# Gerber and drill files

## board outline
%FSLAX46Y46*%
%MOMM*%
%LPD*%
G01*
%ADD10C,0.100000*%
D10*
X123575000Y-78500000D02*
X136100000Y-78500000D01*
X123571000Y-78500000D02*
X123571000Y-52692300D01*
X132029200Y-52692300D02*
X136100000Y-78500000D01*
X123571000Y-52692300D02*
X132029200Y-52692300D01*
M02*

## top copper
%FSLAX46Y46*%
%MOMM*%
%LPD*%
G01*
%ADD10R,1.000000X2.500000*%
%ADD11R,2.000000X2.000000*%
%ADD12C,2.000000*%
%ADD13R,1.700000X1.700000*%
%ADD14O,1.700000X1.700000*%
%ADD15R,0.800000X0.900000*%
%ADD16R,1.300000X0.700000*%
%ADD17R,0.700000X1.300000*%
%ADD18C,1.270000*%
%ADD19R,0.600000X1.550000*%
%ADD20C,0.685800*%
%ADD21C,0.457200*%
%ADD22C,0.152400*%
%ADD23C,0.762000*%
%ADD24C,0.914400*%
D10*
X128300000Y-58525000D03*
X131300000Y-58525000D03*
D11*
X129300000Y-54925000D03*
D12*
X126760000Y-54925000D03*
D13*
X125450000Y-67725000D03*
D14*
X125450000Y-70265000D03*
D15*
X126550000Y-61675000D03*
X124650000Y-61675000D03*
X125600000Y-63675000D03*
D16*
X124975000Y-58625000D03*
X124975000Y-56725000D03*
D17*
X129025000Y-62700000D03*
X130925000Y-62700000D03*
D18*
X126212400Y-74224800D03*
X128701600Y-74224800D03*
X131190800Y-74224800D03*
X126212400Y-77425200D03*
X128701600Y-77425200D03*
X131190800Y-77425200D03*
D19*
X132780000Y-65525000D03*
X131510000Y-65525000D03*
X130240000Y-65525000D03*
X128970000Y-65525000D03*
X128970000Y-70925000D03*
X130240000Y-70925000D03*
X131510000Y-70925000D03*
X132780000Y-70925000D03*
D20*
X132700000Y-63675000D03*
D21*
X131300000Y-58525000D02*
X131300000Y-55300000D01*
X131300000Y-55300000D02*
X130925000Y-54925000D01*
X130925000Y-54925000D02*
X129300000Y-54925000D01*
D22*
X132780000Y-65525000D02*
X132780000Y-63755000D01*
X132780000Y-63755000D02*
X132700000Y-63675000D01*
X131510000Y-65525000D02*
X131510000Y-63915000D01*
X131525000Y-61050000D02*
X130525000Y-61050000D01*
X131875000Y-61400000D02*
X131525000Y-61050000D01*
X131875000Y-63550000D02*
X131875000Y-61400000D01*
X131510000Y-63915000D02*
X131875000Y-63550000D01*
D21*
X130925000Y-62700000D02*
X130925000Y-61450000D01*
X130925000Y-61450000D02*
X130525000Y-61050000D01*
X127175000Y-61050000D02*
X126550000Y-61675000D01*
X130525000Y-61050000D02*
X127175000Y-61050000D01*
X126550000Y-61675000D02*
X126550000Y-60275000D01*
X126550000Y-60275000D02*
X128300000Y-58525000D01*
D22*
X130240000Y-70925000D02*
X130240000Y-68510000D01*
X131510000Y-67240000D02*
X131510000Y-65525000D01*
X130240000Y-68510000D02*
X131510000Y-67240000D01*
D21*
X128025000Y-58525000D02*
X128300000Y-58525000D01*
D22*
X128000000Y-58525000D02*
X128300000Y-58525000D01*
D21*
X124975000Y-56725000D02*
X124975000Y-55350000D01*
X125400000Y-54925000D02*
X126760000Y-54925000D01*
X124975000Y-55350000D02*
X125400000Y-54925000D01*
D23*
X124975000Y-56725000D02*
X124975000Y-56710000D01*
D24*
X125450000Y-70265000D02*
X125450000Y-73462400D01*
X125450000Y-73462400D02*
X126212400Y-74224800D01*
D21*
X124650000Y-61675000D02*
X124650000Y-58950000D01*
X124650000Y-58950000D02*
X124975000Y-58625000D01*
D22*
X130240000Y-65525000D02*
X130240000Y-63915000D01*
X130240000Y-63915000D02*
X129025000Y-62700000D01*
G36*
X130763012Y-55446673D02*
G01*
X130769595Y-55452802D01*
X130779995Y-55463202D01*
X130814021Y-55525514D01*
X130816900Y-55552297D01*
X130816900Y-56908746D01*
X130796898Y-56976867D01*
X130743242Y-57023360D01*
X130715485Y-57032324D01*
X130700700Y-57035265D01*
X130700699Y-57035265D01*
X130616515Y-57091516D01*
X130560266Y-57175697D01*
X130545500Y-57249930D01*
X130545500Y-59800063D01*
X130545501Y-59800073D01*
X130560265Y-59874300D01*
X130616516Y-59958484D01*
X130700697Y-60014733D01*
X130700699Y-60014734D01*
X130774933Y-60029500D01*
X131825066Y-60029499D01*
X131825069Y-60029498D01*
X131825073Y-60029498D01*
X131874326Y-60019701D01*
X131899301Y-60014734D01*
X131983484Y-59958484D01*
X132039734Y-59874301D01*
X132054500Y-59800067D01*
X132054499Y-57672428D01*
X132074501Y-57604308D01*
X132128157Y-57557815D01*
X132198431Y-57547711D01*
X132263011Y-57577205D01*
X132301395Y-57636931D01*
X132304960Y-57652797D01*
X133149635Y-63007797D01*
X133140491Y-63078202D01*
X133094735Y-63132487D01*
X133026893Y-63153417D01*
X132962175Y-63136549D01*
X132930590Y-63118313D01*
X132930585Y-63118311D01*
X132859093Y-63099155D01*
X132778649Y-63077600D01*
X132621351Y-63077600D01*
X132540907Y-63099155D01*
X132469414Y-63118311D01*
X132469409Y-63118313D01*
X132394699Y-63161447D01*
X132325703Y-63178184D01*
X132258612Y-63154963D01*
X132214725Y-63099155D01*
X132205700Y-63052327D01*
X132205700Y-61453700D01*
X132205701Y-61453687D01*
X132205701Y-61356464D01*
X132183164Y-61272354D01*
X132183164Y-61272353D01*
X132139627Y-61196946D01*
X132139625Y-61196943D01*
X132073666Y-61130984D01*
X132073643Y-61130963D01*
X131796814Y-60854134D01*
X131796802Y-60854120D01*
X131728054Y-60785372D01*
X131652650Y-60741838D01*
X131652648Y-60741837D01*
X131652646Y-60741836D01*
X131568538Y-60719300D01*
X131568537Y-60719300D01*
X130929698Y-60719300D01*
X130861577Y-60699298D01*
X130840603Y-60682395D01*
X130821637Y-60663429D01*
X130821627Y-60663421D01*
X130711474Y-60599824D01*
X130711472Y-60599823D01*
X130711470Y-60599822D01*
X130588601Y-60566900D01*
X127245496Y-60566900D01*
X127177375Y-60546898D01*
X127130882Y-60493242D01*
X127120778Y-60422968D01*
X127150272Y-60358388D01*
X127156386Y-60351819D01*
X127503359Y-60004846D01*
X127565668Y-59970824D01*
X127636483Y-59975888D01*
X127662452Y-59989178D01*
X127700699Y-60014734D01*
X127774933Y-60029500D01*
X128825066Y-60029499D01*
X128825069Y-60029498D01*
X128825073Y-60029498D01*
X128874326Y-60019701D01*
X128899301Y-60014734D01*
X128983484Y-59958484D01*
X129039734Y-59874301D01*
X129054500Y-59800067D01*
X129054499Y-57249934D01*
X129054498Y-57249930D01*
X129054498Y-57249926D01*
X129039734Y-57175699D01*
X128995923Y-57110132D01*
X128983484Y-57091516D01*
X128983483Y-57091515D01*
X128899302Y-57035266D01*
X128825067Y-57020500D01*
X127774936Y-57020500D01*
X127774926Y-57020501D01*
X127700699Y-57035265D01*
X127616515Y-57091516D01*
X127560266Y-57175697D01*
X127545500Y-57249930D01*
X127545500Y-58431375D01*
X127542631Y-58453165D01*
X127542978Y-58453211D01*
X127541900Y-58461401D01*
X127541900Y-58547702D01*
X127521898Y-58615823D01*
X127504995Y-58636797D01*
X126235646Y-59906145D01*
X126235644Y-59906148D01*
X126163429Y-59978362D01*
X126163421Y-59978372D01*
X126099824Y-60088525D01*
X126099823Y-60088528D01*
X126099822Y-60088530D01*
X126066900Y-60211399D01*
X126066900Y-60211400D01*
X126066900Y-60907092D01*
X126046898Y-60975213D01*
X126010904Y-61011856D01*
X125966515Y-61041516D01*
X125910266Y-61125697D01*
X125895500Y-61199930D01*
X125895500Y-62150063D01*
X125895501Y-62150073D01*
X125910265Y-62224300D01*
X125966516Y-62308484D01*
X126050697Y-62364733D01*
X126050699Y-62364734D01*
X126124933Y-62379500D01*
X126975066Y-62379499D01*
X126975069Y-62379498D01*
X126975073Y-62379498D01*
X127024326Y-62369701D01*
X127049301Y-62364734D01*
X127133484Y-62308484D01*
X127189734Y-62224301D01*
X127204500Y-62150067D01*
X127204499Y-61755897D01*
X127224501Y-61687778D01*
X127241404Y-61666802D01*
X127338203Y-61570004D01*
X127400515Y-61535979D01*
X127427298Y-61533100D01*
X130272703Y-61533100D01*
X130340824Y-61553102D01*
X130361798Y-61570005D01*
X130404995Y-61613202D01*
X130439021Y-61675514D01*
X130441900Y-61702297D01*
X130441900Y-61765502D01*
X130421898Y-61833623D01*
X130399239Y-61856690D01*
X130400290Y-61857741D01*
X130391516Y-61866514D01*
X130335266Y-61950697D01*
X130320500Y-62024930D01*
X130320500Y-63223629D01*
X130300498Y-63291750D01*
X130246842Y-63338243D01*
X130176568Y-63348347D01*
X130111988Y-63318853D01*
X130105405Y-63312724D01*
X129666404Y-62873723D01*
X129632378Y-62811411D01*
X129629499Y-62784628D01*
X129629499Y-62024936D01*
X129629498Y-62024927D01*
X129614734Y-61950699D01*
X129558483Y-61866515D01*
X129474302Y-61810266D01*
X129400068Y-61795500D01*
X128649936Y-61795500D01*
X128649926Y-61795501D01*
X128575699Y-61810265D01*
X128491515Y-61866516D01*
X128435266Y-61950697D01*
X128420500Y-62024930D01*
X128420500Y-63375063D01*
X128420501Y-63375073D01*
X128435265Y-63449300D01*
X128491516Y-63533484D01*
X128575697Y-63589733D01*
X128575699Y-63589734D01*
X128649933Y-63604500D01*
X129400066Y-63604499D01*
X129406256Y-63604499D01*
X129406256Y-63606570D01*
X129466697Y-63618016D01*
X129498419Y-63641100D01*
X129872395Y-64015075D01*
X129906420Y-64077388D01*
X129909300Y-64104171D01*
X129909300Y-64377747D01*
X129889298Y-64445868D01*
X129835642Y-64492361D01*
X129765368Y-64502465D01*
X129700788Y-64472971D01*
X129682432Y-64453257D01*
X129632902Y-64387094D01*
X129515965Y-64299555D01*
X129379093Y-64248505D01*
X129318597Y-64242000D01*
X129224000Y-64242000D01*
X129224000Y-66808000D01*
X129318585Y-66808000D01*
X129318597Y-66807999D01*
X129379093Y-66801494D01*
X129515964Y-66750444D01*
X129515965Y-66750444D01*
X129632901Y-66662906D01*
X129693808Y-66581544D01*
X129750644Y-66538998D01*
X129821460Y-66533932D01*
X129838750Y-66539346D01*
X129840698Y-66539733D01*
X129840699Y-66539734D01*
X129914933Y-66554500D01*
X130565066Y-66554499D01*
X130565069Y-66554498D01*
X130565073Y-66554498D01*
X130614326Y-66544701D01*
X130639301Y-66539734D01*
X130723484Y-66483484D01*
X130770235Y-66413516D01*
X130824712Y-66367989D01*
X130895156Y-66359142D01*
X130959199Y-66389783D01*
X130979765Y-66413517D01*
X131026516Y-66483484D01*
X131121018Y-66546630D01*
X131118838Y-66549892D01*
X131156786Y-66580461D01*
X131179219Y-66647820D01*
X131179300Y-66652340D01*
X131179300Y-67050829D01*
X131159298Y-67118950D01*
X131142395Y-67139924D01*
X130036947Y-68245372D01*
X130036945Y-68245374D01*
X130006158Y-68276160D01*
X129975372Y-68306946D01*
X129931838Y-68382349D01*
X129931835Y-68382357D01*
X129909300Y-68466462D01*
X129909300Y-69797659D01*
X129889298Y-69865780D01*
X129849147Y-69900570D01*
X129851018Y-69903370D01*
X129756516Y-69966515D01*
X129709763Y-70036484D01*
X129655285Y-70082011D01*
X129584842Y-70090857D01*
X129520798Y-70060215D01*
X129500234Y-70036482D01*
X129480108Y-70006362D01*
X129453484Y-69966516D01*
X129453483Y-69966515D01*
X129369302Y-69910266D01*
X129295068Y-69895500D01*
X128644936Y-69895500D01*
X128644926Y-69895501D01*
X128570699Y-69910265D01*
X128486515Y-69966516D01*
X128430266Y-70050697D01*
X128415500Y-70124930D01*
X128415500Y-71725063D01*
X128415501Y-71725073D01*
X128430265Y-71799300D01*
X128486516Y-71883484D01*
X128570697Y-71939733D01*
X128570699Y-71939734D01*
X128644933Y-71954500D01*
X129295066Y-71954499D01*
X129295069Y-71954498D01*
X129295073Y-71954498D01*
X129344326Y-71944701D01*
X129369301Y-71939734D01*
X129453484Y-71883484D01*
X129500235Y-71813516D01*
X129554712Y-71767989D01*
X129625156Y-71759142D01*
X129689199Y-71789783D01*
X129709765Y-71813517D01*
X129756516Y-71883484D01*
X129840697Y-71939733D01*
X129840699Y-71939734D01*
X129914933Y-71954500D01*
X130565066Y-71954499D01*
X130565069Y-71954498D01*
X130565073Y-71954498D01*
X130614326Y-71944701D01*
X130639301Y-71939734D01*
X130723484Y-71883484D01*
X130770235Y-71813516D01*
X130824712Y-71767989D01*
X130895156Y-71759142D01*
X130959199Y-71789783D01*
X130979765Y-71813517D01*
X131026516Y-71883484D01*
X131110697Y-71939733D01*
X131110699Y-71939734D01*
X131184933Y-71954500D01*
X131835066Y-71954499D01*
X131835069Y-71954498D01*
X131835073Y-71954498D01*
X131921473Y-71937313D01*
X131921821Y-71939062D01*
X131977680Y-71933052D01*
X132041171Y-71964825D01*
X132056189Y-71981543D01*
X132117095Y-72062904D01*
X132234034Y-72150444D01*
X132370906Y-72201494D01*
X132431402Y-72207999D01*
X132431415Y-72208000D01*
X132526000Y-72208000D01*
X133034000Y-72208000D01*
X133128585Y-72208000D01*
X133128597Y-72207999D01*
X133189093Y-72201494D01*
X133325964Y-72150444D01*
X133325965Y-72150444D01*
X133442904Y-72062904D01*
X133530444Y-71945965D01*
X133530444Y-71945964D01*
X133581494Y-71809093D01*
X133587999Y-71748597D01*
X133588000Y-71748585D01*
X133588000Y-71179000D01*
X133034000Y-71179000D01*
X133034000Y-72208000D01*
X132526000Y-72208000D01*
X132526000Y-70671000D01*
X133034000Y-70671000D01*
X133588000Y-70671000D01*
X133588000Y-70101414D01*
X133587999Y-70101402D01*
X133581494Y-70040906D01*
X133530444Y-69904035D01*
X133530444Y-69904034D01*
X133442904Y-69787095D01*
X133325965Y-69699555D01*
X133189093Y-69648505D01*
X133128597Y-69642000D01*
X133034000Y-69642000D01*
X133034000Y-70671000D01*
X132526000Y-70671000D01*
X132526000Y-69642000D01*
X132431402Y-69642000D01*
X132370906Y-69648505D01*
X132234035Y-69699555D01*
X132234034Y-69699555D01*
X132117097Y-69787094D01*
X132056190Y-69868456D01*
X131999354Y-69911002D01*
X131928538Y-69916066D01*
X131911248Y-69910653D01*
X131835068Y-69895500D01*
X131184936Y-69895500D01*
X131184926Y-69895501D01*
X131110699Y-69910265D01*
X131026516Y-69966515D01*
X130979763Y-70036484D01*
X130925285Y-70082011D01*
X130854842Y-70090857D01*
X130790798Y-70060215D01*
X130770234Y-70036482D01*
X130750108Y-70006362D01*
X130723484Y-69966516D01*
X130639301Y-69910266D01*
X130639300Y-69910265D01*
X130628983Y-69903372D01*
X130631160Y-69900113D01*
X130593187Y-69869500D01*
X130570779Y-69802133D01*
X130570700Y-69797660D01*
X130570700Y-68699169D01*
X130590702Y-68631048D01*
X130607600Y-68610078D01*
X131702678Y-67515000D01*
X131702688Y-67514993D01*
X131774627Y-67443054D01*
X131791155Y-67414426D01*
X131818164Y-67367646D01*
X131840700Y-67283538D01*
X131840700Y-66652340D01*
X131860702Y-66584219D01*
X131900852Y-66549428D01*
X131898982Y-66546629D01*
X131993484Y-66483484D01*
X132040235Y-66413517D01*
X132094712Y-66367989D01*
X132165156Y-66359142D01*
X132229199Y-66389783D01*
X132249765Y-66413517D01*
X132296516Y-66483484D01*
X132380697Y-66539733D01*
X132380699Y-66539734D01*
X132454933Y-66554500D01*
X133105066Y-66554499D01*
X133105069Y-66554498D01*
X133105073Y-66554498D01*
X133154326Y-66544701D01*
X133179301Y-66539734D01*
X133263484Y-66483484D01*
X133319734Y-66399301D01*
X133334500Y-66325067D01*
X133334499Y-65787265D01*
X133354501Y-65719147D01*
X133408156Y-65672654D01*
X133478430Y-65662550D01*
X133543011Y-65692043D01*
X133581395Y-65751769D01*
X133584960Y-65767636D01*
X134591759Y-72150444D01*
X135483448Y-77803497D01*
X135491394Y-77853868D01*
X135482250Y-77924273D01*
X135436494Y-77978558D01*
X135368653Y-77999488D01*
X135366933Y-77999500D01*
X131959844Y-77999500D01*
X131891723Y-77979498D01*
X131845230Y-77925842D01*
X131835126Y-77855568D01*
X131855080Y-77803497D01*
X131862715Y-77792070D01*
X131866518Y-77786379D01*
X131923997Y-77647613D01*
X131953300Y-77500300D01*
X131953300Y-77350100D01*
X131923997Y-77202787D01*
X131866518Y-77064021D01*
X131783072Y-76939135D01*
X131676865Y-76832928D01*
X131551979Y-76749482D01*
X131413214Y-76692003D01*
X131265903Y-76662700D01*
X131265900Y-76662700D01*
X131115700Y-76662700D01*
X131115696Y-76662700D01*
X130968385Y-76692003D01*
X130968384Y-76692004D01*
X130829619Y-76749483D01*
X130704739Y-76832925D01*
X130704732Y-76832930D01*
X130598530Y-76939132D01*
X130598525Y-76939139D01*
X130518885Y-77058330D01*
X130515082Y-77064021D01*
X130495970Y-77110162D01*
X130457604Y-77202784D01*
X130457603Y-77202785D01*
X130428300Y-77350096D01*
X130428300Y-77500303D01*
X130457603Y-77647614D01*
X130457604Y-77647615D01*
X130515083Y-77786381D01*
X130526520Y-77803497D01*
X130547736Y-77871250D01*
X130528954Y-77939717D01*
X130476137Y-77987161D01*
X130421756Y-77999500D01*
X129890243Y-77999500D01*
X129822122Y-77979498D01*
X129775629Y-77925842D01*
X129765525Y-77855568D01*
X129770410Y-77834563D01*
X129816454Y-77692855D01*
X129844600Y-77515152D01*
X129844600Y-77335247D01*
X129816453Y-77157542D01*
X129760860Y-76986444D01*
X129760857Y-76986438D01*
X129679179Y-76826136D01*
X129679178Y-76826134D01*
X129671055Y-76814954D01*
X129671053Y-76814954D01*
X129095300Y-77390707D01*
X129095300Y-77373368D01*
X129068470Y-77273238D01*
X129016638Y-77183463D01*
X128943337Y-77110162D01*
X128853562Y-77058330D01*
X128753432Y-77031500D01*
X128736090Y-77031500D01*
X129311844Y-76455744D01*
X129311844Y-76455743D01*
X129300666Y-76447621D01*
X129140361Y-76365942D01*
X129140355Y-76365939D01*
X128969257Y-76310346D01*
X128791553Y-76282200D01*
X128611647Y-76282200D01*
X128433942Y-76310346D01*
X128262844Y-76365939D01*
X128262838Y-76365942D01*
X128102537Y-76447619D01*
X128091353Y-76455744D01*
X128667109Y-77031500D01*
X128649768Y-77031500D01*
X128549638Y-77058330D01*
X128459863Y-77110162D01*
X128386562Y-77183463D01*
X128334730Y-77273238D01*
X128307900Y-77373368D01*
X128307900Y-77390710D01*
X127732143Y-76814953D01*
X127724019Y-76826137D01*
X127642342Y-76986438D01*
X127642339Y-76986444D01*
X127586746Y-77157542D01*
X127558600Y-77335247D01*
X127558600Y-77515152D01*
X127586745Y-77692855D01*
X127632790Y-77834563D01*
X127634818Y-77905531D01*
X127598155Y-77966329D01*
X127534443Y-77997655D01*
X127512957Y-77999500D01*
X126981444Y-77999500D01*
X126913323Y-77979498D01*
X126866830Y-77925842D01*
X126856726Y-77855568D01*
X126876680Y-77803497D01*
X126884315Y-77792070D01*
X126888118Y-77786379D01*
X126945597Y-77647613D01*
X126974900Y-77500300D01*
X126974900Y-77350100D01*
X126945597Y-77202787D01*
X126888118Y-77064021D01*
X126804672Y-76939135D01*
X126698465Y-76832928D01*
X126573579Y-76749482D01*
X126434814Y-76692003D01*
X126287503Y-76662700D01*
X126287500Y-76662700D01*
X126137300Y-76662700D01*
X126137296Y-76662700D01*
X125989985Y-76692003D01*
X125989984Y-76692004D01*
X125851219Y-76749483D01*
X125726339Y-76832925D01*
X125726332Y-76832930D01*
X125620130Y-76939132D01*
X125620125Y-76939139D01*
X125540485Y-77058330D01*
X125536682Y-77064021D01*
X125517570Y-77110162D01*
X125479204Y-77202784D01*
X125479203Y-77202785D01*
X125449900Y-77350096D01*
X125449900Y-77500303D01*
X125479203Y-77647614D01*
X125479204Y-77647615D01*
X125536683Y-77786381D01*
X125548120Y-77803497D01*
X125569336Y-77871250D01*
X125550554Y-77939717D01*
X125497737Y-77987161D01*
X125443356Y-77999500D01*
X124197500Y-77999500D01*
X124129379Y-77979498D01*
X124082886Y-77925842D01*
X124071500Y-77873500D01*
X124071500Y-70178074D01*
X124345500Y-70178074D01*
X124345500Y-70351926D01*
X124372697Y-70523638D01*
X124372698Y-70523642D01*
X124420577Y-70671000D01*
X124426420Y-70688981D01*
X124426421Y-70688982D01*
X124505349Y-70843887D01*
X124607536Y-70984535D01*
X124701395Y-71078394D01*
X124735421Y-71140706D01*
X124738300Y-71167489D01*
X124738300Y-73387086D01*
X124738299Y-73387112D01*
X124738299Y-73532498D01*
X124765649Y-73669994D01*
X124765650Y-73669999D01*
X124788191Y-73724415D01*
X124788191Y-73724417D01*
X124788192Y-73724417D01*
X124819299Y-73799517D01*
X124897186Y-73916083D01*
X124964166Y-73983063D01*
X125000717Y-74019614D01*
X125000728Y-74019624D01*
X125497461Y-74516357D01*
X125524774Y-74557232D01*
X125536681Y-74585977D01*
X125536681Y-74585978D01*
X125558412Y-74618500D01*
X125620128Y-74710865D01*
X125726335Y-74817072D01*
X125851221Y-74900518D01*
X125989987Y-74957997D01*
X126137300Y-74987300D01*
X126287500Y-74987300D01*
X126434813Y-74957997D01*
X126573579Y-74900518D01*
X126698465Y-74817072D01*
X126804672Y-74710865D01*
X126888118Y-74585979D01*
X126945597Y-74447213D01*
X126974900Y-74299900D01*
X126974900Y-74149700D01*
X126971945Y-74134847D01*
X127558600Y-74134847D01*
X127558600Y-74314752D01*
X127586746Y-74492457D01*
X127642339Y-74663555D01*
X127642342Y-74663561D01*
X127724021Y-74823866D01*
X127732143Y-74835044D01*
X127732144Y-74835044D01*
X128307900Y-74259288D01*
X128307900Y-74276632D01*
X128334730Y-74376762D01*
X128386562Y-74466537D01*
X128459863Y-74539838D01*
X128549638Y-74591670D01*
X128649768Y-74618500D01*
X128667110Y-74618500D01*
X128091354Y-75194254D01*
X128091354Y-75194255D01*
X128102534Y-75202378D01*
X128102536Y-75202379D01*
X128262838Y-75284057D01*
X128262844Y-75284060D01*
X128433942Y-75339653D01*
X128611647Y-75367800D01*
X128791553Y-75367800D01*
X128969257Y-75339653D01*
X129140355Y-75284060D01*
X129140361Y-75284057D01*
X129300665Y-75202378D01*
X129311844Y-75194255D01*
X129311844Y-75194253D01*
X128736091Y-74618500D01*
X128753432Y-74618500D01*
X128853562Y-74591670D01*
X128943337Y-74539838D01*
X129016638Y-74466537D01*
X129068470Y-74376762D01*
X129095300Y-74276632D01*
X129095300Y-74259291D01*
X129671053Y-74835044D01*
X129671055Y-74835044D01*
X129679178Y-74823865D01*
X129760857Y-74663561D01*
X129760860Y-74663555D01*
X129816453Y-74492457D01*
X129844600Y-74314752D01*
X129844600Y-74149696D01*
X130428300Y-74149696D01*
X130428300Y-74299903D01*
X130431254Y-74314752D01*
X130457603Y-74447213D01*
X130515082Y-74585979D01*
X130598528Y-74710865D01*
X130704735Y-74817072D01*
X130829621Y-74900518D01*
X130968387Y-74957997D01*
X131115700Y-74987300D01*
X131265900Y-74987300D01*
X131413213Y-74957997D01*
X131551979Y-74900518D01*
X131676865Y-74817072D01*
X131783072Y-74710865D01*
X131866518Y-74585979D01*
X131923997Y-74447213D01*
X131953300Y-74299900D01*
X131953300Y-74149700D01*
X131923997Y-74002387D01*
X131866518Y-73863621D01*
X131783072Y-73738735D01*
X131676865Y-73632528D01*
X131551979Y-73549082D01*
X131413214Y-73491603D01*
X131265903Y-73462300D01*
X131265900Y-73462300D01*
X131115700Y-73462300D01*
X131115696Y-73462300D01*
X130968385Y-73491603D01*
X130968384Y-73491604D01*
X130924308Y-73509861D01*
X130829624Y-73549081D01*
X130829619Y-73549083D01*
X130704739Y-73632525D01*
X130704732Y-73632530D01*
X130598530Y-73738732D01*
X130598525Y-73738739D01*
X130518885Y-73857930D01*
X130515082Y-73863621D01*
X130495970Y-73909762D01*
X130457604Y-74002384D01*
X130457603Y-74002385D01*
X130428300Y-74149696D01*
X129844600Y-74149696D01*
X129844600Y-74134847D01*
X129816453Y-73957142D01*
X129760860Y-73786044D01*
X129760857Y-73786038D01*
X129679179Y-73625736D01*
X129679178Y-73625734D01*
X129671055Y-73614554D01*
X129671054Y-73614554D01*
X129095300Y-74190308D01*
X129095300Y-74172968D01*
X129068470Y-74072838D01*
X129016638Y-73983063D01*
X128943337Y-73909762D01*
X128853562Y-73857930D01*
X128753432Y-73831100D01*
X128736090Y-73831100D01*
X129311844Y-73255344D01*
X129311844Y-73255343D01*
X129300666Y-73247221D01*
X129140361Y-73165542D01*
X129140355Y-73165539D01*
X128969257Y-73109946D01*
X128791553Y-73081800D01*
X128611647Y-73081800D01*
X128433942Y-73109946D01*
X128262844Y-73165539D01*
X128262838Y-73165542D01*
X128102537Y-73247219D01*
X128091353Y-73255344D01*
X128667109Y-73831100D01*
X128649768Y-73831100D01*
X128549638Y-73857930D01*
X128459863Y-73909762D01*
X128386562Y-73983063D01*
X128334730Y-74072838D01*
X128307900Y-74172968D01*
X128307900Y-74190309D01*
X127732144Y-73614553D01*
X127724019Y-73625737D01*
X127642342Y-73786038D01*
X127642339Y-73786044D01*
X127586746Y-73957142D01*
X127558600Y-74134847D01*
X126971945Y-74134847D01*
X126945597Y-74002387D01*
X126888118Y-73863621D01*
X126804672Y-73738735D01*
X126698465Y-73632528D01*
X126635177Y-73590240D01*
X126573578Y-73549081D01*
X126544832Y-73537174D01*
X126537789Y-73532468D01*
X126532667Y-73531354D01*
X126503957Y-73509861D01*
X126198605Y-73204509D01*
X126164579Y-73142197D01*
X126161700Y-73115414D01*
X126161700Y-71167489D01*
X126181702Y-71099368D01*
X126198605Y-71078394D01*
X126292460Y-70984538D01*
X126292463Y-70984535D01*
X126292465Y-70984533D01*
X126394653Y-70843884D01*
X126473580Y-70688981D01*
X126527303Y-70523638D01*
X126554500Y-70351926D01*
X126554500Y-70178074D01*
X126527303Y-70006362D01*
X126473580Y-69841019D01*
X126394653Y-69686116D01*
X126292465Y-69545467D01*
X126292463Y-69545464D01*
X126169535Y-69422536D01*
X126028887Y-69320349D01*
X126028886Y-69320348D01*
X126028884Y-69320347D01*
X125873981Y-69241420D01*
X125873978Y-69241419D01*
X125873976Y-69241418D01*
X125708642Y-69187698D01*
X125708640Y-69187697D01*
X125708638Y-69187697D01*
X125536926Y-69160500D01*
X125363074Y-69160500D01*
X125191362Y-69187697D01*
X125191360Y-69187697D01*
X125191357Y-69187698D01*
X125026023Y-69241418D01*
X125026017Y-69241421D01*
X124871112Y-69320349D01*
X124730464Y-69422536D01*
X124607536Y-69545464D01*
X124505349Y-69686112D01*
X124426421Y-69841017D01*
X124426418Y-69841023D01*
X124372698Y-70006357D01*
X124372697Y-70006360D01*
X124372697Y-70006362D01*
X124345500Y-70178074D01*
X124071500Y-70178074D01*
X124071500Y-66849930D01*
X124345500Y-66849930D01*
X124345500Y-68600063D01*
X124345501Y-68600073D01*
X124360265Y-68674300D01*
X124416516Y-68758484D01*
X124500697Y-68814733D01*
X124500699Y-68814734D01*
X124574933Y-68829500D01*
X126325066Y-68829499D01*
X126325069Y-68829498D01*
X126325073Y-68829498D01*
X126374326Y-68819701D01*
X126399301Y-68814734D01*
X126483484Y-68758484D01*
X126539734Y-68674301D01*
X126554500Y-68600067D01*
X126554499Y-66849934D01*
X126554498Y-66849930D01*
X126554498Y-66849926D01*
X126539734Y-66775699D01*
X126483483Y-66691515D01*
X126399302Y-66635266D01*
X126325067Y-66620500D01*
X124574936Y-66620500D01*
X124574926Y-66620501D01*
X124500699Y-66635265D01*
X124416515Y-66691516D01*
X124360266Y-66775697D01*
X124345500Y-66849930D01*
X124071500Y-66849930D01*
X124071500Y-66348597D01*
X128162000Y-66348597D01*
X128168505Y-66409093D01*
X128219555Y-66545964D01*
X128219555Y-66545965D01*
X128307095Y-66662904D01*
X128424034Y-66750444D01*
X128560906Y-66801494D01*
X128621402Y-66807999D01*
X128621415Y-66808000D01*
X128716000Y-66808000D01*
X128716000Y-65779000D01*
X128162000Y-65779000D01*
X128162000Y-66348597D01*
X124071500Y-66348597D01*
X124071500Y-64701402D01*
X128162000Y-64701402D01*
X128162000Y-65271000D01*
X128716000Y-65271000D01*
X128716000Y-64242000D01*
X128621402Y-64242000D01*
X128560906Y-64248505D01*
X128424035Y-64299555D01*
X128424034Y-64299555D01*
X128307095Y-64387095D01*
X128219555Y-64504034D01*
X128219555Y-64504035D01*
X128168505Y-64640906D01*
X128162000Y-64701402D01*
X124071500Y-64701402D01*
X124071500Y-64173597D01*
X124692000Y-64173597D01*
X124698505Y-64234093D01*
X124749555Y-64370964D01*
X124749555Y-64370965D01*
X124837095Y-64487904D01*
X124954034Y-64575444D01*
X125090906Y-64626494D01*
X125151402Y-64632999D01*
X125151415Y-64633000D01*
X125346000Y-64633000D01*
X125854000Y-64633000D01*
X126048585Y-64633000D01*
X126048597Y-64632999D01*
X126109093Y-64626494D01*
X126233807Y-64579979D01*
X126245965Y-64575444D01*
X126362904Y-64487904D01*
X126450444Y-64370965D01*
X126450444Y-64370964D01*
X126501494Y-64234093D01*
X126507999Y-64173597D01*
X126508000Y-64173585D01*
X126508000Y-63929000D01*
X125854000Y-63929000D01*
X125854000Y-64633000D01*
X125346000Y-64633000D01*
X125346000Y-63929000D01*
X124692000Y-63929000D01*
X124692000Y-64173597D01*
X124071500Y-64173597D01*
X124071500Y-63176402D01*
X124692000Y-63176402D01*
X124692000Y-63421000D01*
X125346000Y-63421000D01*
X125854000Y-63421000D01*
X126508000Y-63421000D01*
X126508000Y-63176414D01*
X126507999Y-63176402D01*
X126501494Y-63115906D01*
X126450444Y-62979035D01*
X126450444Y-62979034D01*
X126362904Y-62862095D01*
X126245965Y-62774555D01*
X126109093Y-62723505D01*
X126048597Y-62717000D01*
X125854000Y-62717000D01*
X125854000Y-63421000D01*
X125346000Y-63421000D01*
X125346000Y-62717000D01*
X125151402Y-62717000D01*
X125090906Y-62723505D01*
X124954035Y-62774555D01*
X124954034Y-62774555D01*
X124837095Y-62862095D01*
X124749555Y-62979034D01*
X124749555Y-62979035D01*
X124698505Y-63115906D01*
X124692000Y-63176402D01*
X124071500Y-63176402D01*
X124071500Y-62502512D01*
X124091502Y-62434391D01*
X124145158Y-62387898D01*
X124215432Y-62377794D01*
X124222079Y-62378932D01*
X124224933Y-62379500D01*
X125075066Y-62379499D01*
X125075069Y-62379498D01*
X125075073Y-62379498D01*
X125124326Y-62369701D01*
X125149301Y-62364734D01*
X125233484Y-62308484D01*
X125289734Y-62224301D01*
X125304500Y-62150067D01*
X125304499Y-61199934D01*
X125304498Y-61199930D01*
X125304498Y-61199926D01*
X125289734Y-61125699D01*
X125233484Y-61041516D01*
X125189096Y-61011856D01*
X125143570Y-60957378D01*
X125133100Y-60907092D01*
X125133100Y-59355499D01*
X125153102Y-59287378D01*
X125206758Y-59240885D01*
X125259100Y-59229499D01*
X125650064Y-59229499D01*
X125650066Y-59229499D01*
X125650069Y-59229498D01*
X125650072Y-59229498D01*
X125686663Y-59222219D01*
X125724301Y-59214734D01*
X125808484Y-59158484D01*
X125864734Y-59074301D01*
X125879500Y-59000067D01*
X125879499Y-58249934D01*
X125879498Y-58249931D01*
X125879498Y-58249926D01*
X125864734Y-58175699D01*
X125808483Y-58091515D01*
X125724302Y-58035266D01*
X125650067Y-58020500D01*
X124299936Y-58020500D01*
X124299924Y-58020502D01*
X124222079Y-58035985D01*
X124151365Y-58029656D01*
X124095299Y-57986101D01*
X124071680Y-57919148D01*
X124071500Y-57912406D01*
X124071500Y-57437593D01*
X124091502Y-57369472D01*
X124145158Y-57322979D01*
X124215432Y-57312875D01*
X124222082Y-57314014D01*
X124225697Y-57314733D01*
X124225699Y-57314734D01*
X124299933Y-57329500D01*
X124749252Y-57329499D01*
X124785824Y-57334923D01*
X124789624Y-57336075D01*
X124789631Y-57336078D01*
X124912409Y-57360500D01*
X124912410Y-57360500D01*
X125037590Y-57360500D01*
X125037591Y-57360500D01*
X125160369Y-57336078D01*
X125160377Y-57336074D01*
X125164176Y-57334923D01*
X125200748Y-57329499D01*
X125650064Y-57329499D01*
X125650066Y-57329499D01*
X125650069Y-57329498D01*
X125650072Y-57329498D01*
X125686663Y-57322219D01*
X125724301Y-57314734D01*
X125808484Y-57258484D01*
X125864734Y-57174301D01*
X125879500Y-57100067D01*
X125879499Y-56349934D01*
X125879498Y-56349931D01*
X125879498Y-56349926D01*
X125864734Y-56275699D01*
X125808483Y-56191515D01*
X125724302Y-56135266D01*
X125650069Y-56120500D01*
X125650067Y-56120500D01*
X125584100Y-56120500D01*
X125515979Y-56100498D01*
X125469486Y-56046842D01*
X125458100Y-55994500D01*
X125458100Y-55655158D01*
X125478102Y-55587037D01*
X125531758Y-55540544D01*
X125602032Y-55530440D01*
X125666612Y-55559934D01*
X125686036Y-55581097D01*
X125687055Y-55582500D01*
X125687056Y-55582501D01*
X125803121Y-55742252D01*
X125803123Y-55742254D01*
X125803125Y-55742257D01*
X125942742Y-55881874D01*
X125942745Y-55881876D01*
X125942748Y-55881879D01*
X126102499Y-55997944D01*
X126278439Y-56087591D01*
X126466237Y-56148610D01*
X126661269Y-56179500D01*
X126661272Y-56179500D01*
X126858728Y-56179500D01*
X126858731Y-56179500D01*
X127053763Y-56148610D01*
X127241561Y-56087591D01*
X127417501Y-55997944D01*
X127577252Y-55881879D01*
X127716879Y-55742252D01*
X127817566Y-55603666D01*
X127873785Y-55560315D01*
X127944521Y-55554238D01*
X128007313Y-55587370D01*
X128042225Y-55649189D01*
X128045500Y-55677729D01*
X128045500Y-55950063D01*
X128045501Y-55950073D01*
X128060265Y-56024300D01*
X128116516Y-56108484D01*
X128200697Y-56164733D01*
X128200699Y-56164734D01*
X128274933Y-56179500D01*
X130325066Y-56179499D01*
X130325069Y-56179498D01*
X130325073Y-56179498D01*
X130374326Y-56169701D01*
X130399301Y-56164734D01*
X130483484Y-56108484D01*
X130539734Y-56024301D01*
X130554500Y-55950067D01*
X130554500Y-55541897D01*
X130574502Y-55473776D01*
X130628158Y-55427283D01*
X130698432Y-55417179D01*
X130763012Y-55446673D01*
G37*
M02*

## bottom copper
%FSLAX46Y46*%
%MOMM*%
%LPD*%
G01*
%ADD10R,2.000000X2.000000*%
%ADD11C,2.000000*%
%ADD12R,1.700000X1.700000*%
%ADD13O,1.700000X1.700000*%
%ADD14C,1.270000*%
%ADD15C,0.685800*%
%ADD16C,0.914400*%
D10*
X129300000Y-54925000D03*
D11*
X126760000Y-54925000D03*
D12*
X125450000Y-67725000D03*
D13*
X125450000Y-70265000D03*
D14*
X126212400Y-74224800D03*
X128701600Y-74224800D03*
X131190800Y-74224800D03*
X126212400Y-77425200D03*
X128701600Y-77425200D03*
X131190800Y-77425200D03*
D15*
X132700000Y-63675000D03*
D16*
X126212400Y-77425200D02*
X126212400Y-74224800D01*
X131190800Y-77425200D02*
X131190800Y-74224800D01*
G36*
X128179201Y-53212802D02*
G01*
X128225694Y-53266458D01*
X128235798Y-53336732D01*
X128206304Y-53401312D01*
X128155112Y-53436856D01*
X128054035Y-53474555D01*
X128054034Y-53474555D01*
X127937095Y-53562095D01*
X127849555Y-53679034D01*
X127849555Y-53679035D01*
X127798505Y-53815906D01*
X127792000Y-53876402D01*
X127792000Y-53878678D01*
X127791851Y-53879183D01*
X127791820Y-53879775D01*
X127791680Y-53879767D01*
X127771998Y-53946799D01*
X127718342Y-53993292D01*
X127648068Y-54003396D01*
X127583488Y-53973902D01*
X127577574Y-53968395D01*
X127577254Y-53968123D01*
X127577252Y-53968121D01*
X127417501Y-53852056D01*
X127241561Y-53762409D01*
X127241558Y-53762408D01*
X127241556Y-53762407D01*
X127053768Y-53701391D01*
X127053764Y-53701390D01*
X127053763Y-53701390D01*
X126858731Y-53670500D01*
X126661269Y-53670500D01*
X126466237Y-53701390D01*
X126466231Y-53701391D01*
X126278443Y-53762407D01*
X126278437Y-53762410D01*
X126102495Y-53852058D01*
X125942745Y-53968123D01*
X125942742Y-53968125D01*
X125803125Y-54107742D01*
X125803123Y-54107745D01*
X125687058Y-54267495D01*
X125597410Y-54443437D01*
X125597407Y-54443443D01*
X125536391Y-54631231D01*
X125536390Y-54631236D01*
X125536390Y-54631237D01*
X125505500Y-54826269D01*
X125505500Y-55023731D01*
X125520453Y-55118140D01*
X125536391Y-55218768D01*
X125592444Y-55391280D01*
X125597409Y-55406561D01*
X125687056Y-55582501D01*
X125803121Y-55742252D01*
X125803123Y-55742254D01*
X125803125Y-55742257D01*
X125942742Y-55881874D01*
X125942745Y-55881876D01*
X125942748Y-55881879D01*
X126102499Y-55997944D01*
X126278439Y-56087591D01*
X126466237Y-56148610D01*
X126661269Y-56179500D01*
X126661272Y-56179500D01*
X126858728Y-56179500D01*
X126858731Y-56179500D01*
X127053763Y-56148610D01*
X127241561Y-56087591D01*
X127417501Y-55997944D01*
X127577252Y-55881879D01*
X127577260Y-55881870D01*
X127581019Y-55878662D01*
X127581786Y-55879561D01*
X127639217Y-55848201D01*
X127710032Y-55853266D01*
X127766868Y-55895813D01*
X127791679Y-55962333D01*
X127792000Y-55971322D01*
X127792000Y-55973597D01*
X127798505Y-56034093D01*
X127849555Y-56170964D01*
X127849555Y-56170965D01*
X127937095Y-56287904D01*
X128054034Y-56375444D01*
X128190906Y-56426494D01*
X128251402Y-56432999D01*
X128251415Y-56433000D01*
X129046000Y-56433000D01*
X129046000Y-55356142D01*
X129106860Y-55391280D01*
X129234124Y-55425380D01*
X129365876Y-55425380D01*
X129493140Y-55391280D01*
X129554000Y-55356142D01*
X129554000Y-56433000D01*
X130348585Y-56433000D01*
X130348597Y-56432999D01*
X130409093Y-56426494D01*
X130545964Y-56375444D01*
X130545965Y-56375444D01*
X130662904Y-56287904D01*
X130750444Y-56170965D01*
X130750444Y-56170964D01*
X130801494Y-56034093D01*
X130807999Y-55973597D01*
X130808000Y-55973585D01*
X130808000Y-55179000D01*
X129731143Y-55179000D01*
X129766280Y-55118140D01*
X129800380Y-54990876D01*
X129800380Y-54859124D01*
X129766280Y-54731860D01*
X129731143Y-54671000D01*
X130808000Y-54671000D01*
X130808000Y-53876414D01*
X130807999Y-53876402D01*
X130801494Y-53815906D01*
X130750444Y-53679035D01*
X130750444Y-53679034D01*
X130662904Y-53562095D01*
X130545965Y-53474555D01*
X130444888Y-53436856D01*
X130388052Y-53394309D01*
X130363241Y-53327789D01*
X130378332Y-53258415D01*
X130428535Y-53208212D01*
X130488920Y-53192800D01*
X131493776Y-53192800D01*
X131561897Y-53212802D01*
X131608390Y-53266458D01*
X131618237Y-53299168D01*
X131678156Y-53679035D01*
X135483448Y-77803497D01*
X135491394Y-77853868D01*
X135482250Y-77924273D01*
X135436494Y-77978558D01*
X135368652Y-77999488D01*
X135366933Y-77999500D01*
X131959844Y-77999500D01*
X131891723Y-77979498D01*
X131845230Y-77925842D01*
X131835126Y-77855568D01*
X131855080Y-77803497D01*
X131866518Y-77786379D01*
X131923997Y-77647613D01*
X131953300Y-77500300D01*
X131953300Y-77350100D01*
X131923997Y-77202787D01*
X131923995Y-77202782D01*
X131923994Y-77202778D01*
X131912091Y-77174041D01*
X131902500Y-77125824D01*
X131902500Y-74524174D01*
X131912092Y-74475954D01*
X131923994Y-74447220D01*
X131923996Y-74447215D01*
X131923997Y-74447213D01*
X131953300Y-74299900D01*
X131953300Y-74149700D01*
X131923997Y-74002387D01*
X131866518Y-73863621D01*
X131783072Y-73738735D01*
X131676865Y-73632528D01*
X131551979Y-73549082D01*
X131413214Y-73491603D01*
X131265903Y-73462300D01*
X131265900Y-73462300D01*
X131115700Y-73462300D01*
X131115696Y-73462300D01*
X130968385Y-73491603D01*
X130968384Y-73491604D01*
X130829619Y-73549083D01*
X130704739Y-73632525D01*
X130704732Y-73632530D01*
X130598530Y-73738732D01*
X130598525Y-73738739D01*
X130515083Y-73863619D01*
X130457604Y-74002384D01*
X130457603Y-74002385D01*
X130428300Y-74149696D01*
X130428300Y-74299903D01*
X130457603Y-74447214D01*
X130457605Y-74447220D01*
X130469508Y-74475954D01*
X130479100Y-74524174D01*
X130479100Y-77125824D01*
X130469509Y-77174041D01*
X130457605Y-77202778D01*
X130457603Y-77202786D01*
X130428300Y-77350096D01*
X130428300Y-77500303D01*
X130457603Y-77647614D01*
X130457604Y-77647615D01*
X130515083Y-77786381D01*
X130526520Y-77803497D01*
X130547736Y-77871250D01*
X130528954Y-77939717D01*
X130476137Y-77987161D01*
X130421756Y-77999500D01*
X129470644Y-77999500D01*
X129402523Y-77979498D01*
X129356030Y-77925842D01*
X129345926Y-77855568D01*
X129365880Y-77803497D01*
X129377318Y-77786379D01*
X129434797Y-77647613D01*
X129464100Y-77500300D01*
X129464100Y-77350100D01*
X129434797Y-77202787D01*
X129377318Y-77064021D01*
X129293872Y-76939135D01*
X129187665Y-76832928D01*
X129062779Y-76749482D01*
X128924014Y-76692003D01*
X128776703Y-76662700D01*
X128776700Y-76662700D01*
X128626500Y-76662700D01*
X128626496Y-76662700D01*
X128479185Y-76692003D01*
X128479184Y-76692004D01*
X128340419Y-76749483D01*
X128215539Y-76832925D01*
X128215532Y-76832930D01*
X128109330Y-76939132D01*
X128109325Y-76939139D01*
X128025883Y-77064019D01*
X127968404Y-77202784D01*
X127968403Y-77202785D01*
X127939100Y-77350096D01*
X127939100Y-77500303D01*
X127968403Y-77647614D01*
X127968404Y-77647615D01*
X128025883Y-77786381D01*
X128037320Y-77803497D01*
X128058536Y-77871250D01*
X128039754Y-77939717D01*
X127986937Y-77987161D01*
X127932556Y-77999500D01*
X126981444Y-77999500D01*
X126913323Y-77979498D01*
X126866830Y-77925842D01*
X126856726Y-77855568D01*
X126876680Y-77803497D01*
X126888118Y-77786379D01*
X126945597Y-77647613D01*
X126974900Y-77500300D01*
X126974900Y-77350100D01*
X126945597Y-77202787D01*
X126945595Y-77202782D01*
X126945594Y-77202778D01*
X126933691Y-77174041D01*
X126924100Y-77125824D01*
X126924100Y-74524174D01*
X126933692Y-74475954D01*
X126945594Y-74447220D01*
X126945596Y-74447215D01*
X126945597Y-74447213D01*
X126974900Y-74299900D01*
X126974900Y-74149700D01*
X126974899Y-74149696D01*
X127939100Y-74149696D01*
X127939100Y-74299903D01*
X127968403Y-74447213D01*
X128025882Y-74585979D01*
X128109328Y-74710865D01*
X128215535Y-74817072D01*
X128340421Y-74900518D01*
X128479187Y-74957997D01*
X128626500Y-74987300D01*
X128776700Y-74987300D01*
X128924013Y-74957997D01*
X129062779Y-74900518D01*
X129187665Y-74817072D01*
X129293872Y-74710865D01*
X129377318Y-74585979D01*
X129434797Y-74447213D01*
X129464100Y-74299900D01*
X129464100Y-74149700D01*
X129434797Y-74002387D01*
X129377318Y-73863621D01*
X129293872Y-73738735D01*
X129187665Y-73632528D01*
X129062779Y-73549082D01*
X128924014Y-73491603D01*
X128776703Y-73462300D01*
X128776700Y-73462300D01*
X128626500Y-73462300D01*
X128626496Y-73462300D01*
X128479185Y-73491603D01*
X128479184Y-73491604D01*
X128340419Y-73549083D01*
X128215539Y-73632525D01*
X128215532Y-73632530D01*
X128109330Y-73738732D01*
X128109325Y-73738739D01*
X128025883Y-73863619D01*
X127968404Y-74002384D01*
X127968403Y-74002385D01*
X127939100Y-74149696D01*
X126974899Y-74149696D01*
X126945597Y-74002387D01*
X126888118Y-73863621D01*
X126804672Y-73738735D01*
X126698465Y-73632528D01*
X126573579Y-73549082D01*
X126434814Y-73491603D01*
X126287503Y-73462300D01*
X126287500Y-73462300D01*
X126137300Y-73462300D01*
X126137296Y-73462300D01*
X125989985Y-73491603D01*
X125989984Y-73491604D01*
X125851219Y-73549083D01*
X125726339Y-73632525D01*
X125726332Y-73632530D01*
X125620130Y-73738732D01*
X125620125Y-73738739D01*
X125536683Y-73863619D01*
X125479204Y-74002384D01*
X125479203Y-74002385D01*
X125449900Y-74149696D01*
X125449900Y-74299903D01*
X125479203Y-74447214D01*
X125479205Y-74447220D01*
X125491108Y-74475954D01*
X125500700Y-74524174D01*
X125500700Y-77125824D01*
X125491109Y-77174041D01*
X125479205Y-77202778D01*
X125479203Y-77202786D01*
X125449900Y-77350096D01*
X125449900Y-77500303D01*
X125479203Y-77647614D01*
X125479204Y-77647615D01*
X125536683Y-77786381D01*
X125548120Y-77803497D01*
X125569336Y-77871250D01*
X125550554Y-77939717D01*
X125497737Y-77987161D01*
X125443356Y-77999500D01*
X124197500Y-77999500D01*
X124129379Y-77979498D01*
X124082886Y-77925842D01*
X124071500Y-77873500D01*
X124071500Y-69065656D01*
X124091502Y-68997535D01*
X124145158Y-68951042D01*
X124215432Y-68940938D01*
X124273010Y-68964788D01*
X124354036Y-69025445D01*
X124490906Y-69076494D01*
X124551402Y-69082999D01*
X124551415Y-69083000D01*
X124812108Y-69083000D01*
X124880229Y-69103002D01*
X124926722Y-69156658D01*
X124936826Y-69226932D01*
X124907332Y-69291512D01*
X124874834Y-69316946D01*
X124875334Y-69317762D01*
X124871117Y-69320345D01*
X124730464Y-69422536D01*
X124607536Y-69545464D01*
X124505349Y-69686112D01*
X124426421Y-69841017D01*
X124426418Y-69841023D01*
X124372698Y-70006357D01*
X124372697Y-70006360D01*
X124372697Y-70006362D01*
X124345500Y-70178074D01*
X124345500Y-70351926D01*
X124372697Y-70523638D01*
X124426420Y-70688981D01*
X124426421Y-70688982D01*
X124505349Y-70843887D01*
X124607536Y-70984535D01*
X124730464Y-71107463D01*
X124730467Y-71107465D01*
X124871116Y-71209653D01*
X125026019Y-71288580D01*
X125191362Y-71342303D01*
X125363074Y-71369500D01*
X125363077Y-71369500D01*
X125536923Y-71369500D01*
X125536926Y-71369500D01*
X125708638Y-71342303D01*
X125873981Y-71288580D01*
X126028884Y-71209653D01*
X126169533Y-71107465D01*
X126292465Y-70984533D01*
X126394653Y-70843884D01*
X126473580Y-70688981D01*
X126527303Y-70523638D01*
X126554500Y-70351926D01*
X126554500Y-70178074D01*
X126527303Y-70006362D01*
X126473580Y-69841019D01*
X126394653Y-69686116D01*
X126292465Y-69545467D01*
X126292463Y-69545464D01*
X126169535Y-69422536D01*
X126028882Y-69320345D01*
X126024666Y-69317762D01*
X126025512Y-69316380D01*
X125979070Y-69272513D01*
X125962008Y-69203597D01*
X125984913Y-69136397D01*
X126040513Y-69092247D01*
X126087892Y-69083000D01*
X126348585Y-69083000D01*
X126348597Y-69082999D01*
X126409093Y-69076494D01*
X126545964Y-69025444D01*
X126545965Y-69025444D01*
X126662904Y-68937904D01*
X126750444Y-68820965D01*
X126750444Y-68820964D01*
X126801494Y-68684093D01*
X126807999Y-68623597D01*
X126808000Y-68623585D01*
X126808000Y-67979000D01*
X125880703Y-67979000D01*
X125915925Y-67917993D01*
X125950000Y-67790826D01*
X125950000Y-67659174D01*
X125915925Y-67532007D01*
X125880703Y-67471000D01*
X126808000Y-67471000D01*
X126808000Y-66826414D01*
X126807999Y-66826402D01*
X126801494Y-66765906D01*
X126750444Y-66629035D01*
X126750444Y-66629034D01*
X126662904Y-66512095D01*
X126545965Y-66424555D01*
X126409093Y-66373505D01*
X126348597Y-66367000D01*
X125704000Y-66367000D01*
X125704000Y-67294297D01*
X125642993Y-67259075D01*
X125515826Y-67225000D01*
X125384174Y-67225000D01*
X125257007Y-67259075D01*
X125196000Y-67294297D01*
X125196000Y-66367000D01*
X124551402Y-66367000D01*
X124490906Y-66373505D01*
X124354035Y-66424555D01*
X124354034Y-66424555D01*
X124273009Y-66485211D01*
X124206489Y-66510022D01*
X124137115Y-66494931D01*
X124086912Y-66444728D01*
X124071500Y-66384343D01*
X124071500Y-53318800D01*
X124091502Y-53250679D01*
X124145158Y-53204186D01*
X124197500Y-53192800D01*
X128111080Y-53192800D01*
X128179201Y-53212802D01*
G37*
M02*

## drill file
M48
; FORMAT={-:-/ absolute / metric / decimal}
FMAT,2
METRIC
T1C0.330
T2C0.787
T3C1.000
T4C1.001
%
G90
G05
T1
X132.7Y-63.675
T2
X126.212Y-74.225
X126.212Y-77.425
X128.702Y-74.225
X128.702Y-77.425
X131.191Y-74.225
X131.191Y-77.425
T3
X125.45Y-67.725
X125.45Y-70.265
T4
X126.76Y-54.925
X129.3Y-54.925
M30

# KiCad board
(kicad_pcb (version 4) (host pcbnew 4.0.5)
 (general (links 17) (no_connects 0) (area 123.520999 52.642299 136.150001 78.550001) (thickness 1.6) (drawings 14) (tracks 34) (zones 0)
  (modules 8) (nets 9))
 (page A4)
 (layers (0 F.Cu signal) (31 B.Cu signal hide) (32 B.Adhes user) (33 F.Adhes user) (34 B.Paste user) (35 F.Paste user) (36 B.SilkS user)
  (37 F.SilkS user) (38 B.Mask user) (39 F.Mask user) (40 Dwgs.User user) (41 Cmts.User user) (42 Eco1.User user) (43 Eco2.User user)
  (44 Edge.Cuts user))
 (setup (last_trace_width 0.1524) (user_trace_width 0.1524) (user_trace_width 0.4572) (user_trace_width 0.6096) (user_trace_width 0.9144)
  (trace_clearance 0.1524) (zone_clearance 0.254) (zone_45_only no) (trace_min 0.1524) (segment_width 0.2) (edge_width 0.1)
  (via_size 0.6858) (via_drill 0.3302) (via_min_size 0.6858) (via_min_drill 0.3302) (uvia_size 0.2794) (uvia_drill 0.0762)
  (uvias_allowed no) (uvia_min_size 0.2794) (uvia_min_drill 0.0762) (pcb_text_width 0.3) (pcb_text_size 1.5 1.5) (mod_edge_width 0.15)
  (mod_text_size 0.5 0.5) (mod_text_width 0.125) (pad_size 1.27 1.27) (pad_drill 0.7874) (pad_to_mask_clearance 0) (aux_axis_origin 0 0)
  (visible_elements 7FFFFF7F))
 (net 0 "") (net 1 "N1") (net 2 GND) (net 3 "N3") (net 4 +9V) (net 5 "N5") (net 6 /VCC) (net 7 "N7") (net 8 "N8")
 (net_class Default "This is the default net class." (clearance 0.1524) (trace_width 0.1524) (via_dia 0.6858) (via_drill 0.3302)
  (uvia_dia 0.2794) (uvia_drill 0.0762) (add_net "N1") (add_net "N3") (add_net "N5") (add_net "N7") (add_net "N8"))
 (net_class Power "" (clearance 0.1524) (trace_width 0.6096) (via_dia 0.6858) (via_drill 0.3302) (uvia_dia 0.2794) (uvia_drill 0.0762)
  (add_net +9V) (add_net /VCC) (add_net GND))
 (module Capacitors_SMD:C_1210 (layer F.Cu) (at 129.8 58.525)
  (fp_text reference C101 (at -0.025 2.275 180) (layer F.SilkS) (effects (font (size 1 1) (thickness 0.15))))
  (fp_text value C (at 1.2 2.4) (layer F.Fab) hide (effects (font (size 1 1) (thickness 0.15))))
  (pad 1 smd rect (at -1.5 0) (size 1 2.5) (layers F.Cu F.Paste F.Mask) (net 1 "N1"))
  (pad 2 smd rect (at 1.5 0) (size 1 2.5) (layers F.Cu F.Paste F.Mask) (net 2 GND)))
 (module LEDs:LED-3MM (layer F.Cu) (at 129.3 54.925 180)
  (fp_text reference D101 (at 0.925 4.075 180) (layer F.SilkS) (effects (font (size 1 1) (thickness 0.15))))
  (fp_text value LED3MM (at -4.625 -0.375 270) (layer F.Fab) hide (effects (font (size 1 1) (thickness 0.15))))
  (pad 1 thru_hole rect (at 0 0 270) (size 2 2) (drill 1.00076) (layers *.Cu *.Mask) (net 2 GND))
  (pad 2 thru_hole circle (at 2.54 0 180) (size 2 2) (drill 1.00076) (layers *.Cu *.Mask) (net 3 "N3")))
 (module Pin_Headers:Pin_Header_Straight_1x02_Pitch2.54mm (layer F.Cu) (at 125.45 67.725)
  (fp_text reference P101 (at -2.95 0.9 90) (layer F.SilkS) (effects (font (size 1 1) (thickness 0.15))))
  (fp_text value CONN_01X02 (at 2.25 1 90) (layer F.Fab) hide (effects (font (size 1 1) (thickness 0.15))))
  (pad 1 thru_hole rect (at 0 0) (size 1.7 1.7) (drill 1) (layers *.Cu *.Mask) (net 2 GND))
  (pad 2 thru_hole oval (at 0 2.54) (size 1.7 1.7) (drill 1) (layers *.Cu *.Mask) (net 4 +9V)))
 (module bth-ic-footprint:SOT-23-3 (layer F.Cu) (at 125.6 62.675 270)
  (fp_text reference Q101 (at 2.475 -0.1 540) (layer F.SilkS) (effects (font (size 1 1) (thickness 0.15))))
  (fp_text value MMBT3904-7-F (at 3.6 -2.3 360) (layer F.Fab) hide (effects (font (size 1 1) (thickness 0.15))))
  (pad 1 smd rect (at -1 -0.95 270) (size 0.9 0.8) (layers F.Cu F.Paste F.Mask) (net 1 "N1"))
  (pad 2 smd rect (at -1 0.95 270) (size 0.9 0.8) (layers F.Cu F.Paste F.Mask) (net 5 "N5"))
  (pad 3 smd rect (at 1 0 270) (size 0.9 0.8) (layers F.Cu F.Paste F.Mask) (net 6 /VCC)))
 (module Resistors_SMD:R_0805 (layer F.Cu) (at 124.975 57.675 90)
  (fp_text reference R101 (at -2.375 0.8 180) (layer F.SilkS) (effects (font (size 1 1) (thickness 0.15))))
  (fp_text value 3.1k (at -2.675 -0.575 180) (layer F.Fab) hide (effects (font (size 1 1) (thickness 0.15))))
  (pad 1 smd rect (at -0.95 0 90) (size 0.7 1.3) (layers F.Cu F.Paste F.Mask) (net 5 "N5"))
  (pad 2 smd rect (at 0.95 0 90) (size 0.7 1.3) (layers F.Cu F.Paste F.Mask) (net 3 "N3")))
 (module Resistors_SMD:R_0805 (layer F.Cu) (at 129.975 62.7)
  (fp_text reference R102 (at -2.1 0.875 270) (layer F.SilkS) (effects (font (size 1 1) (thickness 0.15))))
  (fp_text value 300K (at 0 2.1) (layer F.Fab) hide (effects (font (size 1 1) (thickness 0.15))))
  (pad 1 smd rect (at -0.95 0) (size 0.7 1.3) (layers F.Cu F.Paste F.Mask) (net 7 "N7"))
  (pad 2 smd rect (at 0.95 0) (size 0.7 1.3) (layers F.Cu F.Paste F.Mask) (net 1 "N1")))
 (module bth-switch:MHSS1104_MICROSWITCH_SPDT (layer F.Cu) (at 128.6 75.825)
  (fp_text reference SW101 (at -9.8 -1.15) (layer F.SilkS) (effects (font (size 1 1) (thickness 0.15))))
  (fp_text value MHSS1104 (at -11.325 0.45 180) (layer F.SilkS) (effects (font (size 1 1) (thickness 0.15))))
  (pad 1 thru_hole circle (at -2.3876 -1.6002) (size 1.27 1.27) (drill 0.7874) (layers *.Cu *.Mask F.SilkS) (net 4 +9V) (clearance 0.127))
  (pad 3 thru_hole circle (at 0.1016 -1.6002) (size 1.27 1.27) (drill 0.7874) (layers *.Cu *.Mask F.SilkS) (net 6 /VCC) (clearance 0.127))
  (pad 2 thru_hole circle (at 2.5908 -1.6002) (size 1.27 1.27) (drill 0.7874) (layers *.Cu *.Mask F.SilkS) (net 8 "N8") (clearance 0.127))
  (pad 1 thru_hole circle (at -2.3876 1.6002) (size 1.27 1.27) (drill 0.7874) (layers *.Cu *.Mask F.SilkS) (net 4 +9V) (clearance 0.127))
  (pad 3 thru_hole circle (at 0.1016 1.6002) (size 1.27 1.27) (drill 0.7874) (layers *.Cu *.Mask F.SilkS) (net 6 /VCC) (clearance 0.127))
  (pad 2 thru_hole circle (at 2.5908 1.6002) (size 1.27 1.27) (drill 0.7874) (layers *.Cu *.Mask F.SilkS) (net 8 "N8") (clearance 0.127)))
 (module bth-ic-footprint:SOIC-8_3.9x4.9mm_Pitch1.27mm (layer F.Cu) (at 130.875 68.225 270)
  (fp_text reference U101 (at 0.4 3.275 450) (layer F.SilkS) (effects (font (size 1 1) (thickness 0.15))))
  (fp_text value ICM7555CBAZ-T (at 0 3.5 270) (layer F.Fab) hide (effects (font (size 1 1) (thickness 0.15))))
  (pad 1 smd rect (at -2.7 -1.905 270) (size 1.55 0.6) (layers F.Cu F.Paste F.Mask) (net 2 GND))
  (pad 2 smd rect (at -2.7 -0.635 270) (size 1.55 0.6) (layers F.Cu F.Paste F.Mask) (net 1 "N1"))
  (pad 3 smd rect (at -2.7 0.635 270) (size 1.55 0.6) (layers F.Cu F.Paste F.Mask) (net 7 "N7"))
  (pad 4 smd rect (at -2.7 1.905 270) (size 1.55 0.6) (layers F.Cu F.Paste F.Mask) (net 6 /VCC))
  (pad 5 smd rect (at 2.7 1.905 270) (size 1.55 0.6) (layers F.Cu F.Paste F.Mask))
  (pad 6 smd rect (at 2.7 0.635 270) (size 1.55 0.6) (layers F.Cu F.Paste F.Mask) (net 1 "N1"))
  (pad 7 smd rect (at 2.7 -0.635 270) (size 1.55 0.6) (layers F.Cu F.Paste F.Mask))
  (pad 8 smd rect (at 2.7 -1.905 270) (size 1.55 0.6) (layers F.Cu F.Paste F.Mask) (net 6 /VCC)))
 (gr_line (start 123.575 78.5) (end 136.1 78.5) (angle 90) (layer Edge.Cuts) (width 0.1))
 (gr_line (start 123.571 78.5) (end 123.571 52.6923) (angle 90) (layer Edge.Cuts) (width 0.1))
 (gr_line (start 132.0292 52.6923) (end 136.1 78.5) (angle 90) (layer Edge.Cuts) (width 0.1))
 (gr_line (start 123.571 52.6923) (end 132.0292 52.6923) (angle 90) (layer Edge.Cuts) (width 0.1))
 (segment (start 131.3 58.525) (end 131.3 55.3) (width 0.4572) (layer F.Cu) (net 2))
 (segment (start 131.3 55.3) (end 130.925 54.925) (width 0.4572) (layer F.Cu) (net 2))
 (segment (start 130.925 54.925) (end 129.3 54.925) (width 0.4572) (layer F.Cu) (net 2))
 (segment (start 132.78 65.525) (end 132.78 63.755) (width 0.1524) (layer F.Cu) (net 2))
 (via (at 132.7 63.675) (size 0.6858) (drill 0.3302) (layers F.Cu B.Cu) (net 2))
 (segment (start 132.78 63.755) (end 132.7 63.675) (width 0.1524) (layer F.Cu) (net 2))
 (segment (start 131.51 65.525) (end 131.51 63.915) (width 0.1524) (layer F.Cu) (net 1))
 (segment (start 131.525 61.05) (end 130.525 61.05) (width 0.1524) (layer F.Cu) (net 1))
 (segment (start 131.875 61.4) (end 131.525 61.05) (width 0.1524) (layer F.Cu) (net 1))
 (segment (start 131.875 63.55) (end 131.875 61.4) (width 0.1524) (layer F.Cu) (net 1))
 (segment (start 131.51 63.915) (end 131.875 63.55) (width 0.1524) (layer F.Cu) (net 1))
 (segment (start 130.925 62.7) (end 130.925 61.45) (width 0.4572) (layer F.Cu) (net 1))
 (segment (start 130.925 61.45) (end 130.525 61.05) (width 0.4572) (layer F.Cu) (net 1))
 (segment (start 127.175 61.05) (end 126.55 61.675) (width 0.4572) (layer F.Cu) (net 1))
 (segment (start 130.525 61.05) (end 127.175 61.05) (width 0.4572) (layer F.Cu) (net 1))
 (segment (start 126.55 61.675) (end 126.55 60.275) (width 0.4572) (layer F.Cu) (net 1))
 (segment (start 126.55 60.275) (end 128.3 58.525) (width 0.4572) (layer F.Cu) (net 1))
 (segment (start 130.24 70.925) (end 130.24 68.51) (width 0.1524) (layer F.Cu) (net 1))
 (segment (start 131.51 67.24) (end 131.51 65.525) (width 0.1524) (layer F.Cu) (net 1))
 (segment (start 130.24 68.51) (end 131.51 67.24) (width 0.1524) (layer F.Cu) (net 1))
 (segment (start 128.025 58.525) (end 128.3 58.525) (width 0.4572) (layer F.Cu) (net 1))
 (segment (start 128 58.525) (end 128.3 58.525) (width 0.1524) (layer F.Cu) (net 1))
 (segment (start 124.975 56.725) (end 124.975 55.35) (width 0.4572) (layer F.Cu) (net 3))
 (segment (start 125.4 54.925) (end 126.76 54.925) (width 0.4572) (layer F.Cu) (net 3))
 (segment (start 124.975 55.35) (end 125.4 54.925) (width 0.4572) (layer F.Cu) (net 3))
 (segment (start 124.975 56.725) (end 124.975 56.71) (width 0.762) (layer F.Cu) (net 3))
 (segment (start 126.2124 77.4252) (end 126.2124 74.2248) (width 0.9144) (layer B.Cu) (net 4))
 (segment (start 125.45 70.265) (end 125.45 73.4624) (width 0.9144) (layer F.Cu) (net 4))
 (segment (start 125.45 73.4624) (end 126.2124 74.2248) (width 0.9144) (layer F.Cu) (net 4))
 (segment (start 131.1908 77.4252) (end 131.1908 74.2248) (width 0.9144) (layer B.Cu) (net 8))
 (segment (start 124.65 61.675) (end 124.65 58.95) (width 0.4572) (layer F.Cu) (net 5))
 (segment (start 124.65 58.95) (end 124.975 58.625) (width 0.4572) (layer F.Cu) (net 5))
 (segment (start 130.24 65.525) (end 130.24 63.915) (width 0.1524) (layer F.Cu) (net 7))
 (segment (start 130.24 63.915) (end 129.025 62.7) (width 0.1524) (layer F.Cu) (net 7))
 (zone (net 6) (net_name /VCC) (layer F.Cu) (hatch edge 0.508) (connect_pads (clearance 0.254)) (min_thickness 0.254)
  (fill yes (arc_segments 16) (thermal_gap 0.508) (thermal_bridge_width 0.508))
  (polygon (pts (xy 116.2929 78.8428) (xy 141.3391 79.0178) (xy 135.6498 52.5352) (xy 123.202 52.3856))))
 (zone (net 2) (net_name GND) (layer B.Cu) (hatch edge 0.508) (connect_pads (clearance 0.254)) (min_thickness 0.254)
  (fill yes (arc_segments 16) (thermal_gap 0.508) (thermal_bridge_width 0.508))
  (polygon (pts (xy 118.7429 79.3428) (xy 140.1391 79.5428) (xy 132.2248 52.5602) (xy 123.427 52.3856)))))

